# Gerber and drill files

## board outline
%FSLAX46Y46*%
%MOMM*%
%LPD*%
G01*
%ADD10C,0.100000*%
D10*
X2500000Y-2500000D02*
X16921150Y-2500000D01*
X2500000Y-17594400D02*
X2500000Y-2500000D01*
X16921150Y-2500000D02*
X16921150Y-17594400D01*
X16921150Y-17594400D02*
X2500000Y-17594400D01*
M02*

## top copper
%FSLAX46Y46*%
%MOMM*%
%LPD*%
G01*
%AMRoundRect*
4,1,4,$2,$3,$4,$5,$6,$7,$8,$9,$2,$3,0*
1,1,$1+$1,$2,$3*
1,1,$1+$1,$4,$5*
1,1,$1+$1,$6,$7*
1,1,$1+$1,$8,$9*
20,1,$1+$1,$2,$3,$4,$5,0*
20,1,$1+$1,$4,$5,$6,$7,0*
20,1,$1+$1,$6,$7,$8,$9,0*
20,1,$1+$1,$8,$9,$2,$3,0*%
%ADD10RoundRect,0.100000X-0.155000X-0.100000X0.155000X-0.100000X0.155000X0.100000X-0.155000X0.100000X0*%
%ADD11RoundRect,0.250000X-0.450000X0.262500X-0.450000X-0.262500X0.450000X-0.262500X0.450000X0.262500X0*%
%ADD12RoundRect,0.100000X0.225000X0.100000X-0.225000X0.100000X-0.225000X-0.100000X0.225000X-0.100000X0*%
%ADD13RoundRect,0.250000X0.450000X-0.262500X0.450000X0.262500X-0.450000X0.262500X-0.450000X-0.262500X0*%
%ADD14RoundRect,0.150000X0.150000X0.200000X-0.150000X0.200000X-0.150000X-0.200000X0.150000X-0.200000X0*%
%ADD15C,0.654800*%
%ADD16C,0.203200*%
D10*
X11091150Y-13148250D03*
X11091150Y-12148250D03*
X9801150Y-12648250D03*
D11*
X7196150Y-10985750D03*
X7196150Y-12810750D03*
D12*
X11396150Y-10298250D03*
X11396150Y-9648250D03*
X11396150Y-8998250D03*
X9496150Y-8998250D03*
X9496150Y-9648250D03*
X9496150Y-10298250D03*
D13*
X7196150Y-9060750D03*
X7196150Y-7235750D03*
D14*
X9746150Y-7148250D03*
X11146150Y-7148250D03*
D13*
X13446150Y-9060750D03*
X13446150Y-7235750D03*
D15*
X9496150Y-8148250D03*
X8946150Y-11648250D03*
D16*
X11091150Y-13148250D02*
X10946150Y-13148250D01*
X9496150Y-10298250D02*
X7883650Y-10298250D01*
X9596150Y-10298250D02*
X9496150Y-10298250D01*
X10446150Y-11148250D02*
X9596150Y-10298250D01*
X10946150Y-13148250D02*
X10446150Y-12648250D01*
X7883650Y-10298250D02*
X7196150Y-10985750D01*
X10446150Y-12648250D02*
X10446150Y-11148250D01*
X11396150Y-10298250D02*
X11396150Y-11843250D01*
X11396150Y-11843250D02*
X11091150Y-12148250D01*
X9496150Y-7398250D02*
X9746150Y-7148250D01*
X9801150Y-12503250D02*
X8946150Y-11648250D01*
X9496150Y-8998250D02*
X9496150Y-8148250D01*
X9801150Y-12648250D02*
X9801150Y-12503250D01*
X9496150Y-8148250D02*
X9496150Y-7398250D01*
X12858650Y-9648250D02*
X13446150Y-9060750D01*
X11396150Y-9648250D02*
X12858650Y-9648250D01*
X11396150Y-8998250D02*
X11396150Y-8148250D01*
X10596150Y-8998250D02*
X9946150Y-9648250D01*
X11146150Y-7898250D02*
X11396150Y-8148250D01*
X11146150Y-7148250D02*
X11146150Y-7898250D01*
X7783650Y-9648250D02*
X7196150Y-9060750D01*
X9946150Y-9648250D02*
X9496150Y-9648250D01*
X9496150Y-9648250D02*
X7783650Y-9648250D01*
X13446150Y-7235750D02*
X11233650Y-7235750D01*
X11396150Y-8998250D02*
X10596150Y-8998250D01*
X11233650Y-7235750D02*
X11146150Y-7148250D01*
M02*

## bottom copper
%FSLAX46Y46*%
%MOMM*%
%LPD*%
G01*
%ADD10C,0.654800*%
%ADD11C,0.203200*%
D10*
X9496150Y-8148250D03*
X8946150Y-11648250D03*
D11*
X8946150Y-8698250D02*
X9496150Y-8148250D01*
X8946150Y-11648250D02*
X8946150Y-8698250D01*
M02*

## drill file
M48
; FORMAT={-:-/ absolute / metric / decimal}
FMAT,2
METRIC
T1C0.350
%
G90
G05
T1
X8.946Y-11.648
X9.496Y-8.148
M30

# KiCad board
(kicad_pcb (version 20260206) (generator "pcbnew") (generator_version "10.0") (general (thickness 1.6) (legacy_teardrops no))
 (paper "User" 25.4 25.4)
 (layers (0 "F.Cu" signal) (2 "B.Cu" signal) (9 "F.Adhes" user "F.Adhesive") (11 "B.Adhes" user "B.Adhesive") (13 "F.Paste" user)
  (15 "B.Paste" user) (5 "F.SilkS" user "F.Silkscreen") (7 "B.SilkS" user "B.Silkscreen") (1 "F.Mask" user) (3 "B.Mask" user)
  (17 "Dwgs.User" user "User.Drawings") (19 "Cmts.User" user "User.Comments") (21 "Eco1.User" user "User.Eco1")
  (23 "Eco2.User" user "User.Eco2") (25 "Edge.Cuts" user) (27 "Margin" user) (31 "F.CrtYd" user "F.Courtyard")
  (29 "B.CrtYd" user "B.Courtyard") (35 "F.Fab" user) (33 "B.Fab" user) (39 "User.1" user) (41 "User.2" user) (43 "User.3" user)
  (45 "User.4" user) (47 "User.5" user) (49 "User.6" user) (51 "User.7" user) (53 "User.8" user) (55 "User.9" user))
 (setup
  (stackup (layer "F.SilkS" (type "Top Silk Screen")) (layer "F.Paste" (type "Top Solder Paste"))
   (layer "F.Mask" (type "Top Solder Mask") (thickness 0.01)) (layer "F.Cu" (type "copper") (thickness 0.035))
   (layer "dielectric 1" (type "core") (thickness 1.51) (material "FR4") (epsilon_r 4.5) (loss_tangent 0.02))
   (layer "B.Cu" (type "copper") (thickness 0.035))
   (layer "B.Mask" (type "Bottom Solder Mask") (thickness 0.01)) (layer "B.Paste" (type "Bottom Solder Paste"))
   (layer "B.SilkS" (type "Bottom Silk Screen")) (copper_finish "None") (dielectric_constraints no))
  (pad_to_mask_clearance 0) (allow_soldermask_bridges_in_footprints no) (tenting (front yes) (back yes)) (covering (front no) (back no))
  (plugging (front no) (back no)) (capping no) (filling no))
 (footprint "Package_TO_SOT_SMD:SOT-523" (layer "F.Cu") (at 10.44615 12.64825 180)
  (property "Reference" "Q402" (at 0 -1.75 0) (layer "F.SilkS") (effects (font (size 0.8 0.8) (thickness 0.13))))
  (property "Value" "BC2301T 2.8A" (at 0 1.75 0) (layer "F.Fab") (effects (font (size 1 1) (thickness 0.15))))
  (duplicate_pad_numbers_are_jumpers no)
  (pad "1" smd roundrect (at -0.645 -0.5) (size 0.51 0.4) (layers "F.Cu" "F.Mask" "F.Paste") (roundrect_rratio 0.25) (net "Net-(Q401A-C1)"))
  (pad "2" smd roundrect (at -0.645 0.5) (size 0.51 0.4) (layers "F.Cu" "F.Mask" "F.Paste") (roundrect_rratio 0.25) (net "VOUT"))
  (pad "3" smd roundrect (at 0.645 0) (size 0.51 0.4) (layers "F.Cu" "F.Mask" "F.Paste") (roundrect_rratio 0.25) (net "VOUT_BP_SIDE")))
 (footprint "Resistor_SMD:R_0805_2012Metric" (layer "F.Cu") (at 7.19615 11.89825 -90)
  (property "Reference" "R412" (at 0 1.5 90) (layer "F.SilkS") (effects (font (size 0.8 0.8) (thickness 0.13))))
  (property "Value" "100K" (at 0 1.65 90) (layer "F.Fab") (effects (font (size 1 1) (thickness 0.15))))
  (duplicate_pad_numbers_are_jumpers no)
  (pad "1" smd roundrect (at -0.9125 0 270) (size 1.025 1.4) (layers "F.Cu" "F.Mask" "F.Paste") (roundrect_rratio 0.243902)
   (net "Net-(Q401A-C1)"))
  (pad "2" smd roundrect (at 0.9125 0 270) (size 1.025 1.4) (layers "F.Cu" "F.Mask" "F.Paste") (roundrect_rratio 0.243902) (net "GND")))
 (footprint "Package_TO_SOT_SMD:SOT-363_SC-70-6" (layer "F.Cu") (at 10.44615 9.64825 180)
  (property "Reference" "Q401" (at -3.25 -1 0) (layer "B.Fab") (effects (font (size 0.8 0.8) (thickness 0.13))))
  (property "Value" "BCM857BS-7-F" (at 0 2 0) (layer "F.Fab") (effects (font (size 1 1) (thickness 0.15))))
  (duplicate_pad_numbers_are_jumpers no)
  (pad "1" smd roundrect (at -0.95 -0.65 180) (size 0.65 0.4) (layers "F.Cu" "F.Mask" "F.Paste") (roundrect_rratio 0.25) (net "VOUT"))
  (pad "2" smd roundrect (at -0.95 0 180) (size 0.65 0.4) (layers "F.Cu" "F.Mask" "F.Paste") (roundrect_rratio 0.25) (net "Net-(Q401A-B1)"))
  (pad "3" smd roundrect (at -0.95 0.65 180) (size 0.65 0.4) (layers "F.Cu" "F.Mask" "F.Paste") (roundrect_rratio 0.25) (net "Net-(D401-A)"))
  (pad "4" smd roundrect (at 0.95 0.65 180) (size 0.65 0.4) (layers "F.Cu" "F.Mask" "F.Paste") (roundrect_rratio 0.25) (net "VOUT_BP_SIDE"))
  (pad "5" smd roundrect (at 0.95 0 180) (size 0.65 0.4) (layers "F.Cu" "F.Mask" "F.Paste") (roundrect_rratio 0.25) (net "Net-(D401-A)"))
  (pad "6" smd roundrect (at 0.95 -0.65 180) (size 0.65 0.4) (layers "F.Cu" "F.Mask" "F.Paste") (roundrect_rratio 0.25)
   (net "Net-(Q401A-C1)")))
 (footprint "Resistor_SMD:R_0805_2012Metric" (layer "F.Cu") (at 7.19615 8.14825 90)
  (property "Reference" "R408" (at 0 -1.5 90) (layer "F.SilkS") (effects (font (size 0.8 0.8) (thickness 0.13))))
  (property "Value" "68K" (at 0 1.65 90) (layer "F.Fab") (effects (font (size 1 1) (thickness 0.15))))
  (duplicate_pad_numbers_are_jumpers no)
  (pad "1" smd roundrect (at -0.9125 0 90) (size 1.025 1.4) (layers "F.Cu" "F.Mask" "F.Paste") (roundrect_rratio 0.243902)
   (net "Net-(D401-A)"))
  (pad "2" smd roundrect (at 0.9125 0 90) (size 1.025 1.4) (layers "F.Cu" "F.Mask" "F.Paste") (roundrect_rratio 0.243902) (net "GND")))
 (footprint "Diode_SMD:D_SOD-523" (layer "F.Cu") (at 10.44615 7.14825)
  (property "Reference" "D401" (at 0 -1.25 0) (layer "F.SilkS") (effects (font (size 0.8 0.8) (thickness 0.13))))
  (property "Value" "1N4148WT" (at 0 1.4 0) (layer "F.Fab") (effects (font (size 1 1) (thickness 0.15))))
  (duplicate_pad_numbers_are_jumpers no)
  (pad "1" smd roundrect (at -0.7 0 180) (size 0.6 0.7) (layers "F.Cu" "F.Mask" "F.Paste") (roundrect_rratio 0.25) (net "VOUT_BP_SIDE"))
  (pad "2" smd roundrect (at 0.7 0 180) (size 0.6 0.7) (layers "F.Cu" "F.Mask" "F.Paste") (roundrect_rratio 0.25) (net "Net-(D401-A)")))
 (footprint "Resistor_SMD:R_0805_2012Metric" (layer "F.Cu") (at 13.44615 8.14825 90)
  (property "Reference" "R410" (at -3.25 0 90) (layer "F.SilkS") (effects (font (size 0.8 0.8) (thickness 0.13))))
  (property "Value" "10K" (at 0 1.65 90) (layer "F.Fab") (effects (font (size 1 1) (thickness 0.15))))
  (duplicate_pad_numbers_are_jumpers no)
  (pad "1" smd roundrect (at -0.9125 0 90) (size 1.025 1.4) (layers "F.Cu" "F.Mask" "F.Paste") (roundrect_rratio 0.243902)
   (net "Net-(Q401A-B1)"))
  (pad "2" smd roundrect (at 0.9125 0 90) (size 1.025 1.4) (layers "F.Cu" "F.Mask" "F.Paste") (roundrect_rratio 0.243902)
   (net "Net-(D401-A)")))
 (gr_line (start 2.5 2.5) (end 16.92115 2.5) (stroke (width 0.1) (type default)) (layer "Edge.Cuts"))
 (gr_line (start 2.5 17.5944) (end 2.5 2.5) (stroke (width 0.1) (type default)) (layer "Edge.Cuts"))
 (gr_line (start 16.92115 2.5) (end 16.92115 17.5944) (stroke (width 0.1) (type default)) (layer "Edge.Cuts"))
 (gr_line (start 16.92115 17.5944) (end 2.5 17.5944) (stroke (width 0.1) (type default)) (layer "Edge.Cuts"))
 (segment (start 11.09115 13.14825) (end 10.94615 13.14825) (width 0.2032) (layer "F.Cu") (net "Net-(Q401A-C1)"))
 (segment (start 9.49615 10.29825) (end 7.88365 10.29825) (width 0.2032) (layer "F.Cu") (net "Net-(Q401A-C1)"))
 (segment (start 9.59615 10.29825) (end 9.49615 10.29825) (width 0.2032) (layer "F.Cu") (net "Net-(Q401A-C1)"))
 (segment (start 10.44615 11.14825) (end 9.59615 10.29825) (width 0.2032) (layer "F.Cu") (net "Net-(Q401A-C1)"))
 (segment (start 10.94615 13.14825) (end 10.44615 12.64825) (width 0.2032) (layer "F.Cu") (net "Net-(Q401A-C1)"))
 (segment (start 7.88365 10.29825) (end 7.19615 10.98575) (width 0.2032) (layer "F.Cu") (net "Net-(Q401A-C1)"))
 (segment (start 10.44615 12.64825) (end 10.44615 11.14825) (width 0.2032) (layer "F.Cu") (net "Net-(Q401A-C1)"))
 (segment (start 11.39615 10.29825) (end 11.39615 11.84325) (width 0.2032) (layer "F.Cu") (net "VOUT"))
 (segment (start 11.39615 11.84325) (end 11.09115 12.14825) (width 0.2032) (layer "F.Cu") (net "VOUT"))
 (segment (start 9.49615 7.39825) (end 9.74615 7.14825) (width 0.2032) (layer "F.Cu") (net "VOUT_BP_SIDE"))
 (segment (start 9.80115 12.50325) (end 8.94615 11.64825) (width 0.2032) (layer "F.Cu") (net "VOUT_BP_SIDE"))
 (segment (start 9.49615 8.99825) (end 9.49615 8.14825) (width 0.2032) (layer "F.Cu") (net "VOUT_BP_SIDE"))
 (segment (start 9.80115 12.64825) (end 9.80115 12.50325) (width 0.2032) (layer "F.Cu") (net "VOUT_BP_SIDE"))
 (segment (start 9.49615 8.14825) (end 9.49615 7.39825) (width 0.2032) (layer "F.Cu") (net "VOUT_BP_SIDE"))
 (via (at 9.49615 8.14825) (size 0.6548) (drill 0.35) (layers "F.Cu" "B.Cu") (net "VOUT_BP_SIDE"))
 (via (at 8.94615 11.64825) (size 0.6548) (drill 0.35) (layers "F.Cu" "B.Cu") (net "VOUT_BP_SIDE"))
 (segment (start 8.94615 8.69825) (end 9.49615 8.14825) (width 0.2032) (layer "B.Cu") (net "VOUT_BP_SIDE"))
 (segment (start 8.94615 11.64825) (end 8.94615 8.69825) (width 0.2032) (layer "B.Cu") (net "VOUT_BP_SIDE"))
 (segment (start 12.85865 9.64825) (end 13.44615 9.06075) (width 0.2032) (layer "F.Cu") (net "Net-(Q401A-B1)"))
 (segment (start 11.39615 9.64825) (end 12.85865 9.64825) (width 0.2032) (layer "F.Cu") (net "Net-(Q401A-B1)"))
 (segment (start 11.39615 8.99825) (end 11.39615 8.14825) (width 0.2032) (layer "F.Cu") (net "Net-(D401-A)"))
 (segment (start 10.59615 8.99825) (end 9.94615 9.64825) (width 0.2032) (layer "F.Cu") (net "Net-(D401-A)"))
 (segment (start 11.14615 7.89825) (end 11.39615 8.14825) (width 0.2032) (layer "F.Cu") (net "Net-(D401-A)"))
 (segment (start 11.14615 7.14825) (end 11.14615 7.89825) (width 0.2032) (layer "F.Cu") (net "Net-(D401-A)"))
 (segment (start 7.78365 9.64825) (end 7.19615 9.06075) (width 0.2032) (layer "F.Cu") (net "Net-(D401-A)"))
 (segment (start 9.94615 9.64825) (end 9.49615 9.64825) (width 0.2032) (layer "F.Cu") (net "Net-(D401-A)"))
 (segment (start 9.49615 9.64825) (end 7.78365 9.64825) (width 0.2032) (layer "F.Cu") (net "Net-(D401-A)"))
 (segment (start 13.44615 7.23575) (end 11.23365 7.23575) (width 0.2032) (layer "F.Cu") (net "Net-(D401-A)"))
 (segment (start 11.39615 8.99825) (end 10.59615 8.99825) (width 0.2032) (layer "F.Cu") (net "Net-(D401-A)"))
 (segment (start 11.23365 7.23575) (end 11.14615 7.14825) (width 0.2032) (layer "F.Cu") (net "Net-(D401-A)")))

